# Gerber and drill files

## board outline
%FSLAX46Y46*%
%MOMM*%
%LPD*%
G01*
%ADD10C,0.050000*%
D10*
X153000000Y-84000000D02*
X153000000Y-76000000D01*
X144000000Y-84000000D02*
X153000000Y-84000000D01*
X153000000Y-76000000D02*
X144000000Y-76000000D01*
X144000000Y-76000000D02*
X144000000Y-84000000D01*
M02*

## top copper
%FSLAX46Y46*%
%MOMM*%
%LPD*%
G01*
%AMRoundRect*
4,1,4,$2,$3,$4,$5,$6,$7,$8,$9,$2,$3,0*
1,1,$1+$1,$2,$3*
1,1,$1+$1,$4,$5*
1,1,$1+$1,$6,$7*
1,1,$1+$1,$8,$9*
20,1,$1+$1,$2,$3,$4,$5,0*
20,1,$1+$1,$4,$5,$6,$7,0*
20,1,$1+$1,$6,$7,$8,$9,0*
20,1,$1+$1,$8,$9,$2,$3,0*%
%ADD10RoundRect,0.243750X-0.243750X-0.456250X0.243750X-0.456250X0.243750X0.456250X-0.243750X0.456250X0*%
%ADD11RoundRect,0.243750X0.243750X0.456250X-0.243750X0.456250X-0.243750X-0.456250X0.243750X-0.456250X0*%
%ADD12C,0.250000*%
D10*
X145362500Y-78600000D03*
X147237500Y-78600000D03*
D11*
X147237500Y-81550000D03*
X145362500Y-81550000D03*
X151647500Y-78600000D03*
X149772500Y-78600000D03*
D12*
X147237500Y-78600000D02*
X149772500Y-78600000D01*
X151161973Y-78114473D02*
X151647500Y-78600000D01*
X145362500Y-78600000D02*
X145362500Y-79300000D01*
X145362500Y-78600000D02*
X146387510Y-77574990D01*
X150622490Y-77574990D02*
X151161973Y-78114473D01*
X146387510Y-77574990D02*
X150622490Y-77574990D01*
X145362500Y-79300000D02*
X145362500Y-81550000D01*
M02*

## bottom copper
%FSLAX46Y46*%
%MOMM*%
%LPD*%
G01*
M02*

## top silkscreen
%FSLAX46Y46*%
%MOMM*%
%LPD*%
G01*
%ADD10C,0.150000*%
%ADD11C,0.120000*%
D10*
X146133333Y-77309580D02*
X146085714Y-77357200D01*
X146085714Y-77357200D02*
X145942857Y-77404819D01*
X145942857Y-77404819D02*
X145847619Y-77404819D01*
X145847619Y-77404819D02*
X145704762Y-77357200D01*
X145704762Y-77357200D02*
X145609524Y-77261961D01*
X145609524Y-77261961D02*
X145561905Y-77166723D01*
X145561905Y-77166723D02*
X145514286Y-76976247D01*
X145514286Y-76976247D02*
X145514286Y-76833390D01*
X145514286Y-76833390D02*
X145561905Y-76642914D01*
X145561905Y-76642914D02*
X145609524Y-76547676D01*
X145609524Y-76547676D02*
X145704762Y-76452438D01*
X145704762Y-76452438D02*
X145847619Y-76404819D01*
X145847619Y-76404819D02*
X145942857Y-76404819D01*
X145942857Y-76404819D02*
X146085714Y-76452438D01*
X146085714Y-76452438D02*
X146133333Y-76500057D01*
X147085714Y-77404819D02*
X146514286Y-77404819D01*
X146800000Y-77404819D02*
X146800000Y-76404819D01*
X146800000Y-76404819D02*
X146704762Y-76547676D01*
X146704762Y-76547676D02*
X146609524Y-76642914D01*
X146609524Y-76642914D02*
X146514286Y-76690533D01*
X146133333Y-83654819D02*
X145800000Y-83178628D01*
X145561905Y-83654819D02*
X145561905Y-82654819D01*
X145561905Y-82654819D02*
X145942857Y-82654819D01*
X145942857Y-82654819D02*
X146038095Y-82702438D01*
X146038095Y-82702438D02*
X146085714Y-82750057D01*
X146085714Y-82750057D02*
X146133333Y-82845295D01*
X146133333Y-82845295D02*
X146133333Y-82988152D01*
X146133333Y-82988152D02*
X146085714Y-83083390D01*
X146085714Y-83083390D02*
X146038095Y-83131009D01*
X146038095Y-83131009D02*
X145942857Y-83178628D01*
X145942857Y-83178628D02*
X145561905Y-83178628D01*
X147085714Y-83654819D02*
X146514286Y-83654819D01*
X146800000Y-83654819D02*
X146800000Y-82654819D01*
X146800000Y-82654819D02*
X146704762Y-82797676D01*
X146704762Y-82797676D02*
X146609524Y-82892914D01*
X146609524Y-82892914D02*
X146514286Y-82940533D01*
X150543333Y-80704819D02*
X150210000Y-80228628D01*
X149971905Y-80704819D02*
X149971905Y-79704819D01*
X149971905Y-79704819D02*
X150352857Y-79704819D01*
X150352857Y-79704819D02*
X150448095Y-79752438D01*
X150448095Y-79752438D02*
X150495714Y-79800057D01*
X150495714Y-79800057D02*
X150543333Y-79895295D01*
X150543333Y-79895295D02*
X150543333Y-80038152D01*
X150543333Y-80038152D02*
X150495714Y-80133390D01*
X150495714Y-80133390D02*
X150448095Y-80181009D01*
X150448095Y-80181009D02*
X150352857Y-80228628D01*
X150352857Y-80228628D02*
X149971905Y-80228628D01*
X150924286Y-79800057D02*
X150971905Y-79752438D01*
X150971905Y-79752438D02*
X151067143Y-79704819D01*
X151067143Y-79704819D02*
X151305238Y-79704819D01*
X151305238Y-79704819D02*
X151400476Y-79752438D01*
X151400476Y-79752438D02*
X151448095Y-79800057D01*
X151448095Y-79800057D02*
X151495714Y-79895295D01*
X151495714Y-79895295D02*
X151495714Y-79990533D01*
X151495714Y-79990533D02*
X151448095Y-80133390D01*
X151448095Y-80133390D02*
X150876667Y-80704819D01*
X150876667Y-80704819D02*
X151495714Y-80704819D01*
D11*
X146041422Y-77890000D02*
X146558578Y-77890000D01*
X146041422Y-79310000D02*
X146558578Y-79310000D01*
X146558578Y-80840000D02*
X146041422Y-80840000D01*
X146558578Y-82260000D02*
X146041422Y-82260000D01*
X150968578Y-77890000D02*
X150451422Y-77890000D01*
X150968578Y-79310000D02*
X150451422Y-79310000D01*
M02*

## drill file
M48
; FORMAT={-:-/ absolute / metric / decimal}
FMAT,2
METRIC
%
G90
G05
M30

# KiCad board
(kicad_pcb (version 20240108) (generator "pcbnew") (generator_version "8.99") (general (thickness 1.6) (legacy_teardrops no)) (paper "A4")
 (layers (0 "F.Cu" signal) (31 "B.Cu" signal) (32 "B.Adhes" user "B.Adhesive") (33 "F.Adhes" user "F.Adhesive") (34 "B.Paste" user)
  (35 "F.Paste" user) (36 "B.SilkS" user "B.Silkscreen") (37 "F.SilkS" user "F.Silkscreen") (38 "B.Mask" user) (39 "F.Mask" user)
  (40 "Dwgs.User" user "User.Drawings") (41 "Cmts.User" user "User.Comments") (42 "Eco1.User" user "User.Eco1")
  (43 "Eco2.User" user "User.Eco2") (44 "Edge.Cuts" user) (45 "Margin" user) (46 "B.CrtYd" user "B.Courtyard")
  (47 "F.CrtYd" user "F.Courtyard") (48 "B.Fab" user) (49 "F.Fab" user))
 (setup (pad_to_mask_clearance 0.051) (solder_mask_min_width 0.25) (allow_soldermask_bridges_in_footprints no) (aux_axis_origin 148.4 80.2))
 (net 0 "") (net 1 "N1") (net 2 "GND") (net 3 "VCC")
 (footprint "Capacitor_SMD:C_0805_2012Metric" (layer "F.Cu") (at 146.3 78.6)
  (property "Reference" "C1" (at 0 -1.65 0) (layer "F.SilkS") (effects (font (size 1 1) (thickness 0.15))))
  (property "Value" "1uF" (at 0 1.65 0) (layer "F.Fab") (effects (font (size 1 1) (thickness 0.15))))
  (fp_line (start -0.258578 -0.71) (end 0.258578 -0.71) (stroke (width 0.12) (type solid)) (layer "F.SilkS"))
  (fp_line (start -0.258578 0.71) (end 0.258578 0.71) (stroke (width 0.12) (type solid)) (layer "F.SilkS"))
  (pad "1" smd roundrect (at -0.9375 0) (size 0.975 1.4) (layers "F.Cu" "F.Paste" "F.Mask") (roundrect_rratio 0.25) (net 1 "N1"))
  (pad "2" smd roundrect (at 0.9375 0) (size 0.975 1.4) (layers "F.Cu" "F.Paste" "F.Mask") (roundrect_rratio 0.25) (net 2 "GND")))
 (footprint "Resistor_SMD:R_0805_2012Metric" (layer "F.Cu") (at 146.3 81.55 180)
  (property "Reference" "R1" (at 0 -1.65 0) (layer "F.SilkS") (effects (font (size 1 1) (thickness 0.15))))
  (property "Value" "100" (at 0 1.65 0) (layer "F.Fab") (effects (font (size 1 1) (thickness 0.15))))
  (fp_line (start -0.258578 0.71) (end 0.258578 0.71) (stroke (width 0.12) (type solid)) (layer "F.SilkS"))
  (fp_line (start -0.258578 -0.71) (end 0.258578 -0.71) (stroke (width 0.12) (type solid)) (layer "F.SilkS"))
  (pad "1" smd roundrect (at -0.9375 0 180) (size 0.975 1.4) (layers "F.Cu" "F.Paste" "F.Mask") (roundrect_rratio 0.25) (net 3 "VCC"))
  (pad "2" smd roundrect (at 0.9375 0 180) (size 0.975 1.4) (layers "F.Cu" "F.Paste" "F.Mask") (roundrect_rratio 0.25) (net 1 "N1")))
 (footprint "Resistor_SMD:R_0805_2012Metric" (layer "F.Cu") (at 150.71 78.6 180)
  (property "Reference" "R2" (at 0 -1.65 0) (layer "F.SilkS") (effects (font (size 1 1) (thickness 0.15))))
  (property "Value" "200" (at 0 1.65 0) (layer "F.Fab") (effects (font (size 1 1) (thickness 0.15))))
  (fp_line (start -0.258578 0.71) (end 0.258578 0.71) (stroke (width 0.12) (type solid)) (layer "F.SilkS"))
  (fp_line (start -0.258578 -0.71) (end 0.258578 -0.71) (stroke (width 0.12) (type solid)) (layer "F.SilkS"))
  (pad "1" smd roundrect (at -0.9375 0 180) (size 0.975 1.4) (layers "F.Cu" "F.Paste" "F.Mask") (roundrect_rratio 0.25) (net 1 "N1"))
  (pad "2" smd roundrect (at 0.9375 0 180) (size 0.975 1.4) (layers "F.Cu" "F.Paste" "F.Mask") (roundrect_rratio 0.25) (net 2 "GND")))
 (gr_line (start 153 84) (end 153 76) (stroke (width 0.05) (type solid)) (layer "Edge.Cuts"))
 (gr_line (start 144 84) (end 153 84) (stroke (width 0.05) (type solid)) (layer "Edge.Cuts"))
 (gr_line (start 153 76) (end 144 76) (stroke (width 0.05) (type solid)) (layer "Edge.Cuts"))
 (gr_line (start 144 76) (end 144 84) (stroke (width 0.05) (type solid)) (layer "Edge.Cuts"))
 (segment (start 147.2375 78.6) (end 149.7725 78.6) (width 0.25) (layer "F.Cu") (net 2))
 (segment (start 151.161973 78.114473) (end 151.6475 78.6) (width 0.25) (layer "F.Cu") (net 1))
 (segment (start 145.3625 78.6) (end 145.3625 79.3) (width 0.25) (layer "F.Cu") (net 1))
 (segment (start 145.3625 78.6) (end 146.38751 77.57499) (width 0.25) (layer "F.Cu") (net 1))
 (segment (start 150.62249 77.57499) (end 151.161973 78.114473) (width 0.25) (layer "F.Cu") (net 1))
 (segment (start 146.38751 77.57499) (end 150.62249 77.57499) (width 0.25) (layer "F.Cu") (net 1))
 (segment (start 145.3625 79.3) (end 145.3625 81.55) (width 0.25) (layer "F.Cu") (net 1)))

